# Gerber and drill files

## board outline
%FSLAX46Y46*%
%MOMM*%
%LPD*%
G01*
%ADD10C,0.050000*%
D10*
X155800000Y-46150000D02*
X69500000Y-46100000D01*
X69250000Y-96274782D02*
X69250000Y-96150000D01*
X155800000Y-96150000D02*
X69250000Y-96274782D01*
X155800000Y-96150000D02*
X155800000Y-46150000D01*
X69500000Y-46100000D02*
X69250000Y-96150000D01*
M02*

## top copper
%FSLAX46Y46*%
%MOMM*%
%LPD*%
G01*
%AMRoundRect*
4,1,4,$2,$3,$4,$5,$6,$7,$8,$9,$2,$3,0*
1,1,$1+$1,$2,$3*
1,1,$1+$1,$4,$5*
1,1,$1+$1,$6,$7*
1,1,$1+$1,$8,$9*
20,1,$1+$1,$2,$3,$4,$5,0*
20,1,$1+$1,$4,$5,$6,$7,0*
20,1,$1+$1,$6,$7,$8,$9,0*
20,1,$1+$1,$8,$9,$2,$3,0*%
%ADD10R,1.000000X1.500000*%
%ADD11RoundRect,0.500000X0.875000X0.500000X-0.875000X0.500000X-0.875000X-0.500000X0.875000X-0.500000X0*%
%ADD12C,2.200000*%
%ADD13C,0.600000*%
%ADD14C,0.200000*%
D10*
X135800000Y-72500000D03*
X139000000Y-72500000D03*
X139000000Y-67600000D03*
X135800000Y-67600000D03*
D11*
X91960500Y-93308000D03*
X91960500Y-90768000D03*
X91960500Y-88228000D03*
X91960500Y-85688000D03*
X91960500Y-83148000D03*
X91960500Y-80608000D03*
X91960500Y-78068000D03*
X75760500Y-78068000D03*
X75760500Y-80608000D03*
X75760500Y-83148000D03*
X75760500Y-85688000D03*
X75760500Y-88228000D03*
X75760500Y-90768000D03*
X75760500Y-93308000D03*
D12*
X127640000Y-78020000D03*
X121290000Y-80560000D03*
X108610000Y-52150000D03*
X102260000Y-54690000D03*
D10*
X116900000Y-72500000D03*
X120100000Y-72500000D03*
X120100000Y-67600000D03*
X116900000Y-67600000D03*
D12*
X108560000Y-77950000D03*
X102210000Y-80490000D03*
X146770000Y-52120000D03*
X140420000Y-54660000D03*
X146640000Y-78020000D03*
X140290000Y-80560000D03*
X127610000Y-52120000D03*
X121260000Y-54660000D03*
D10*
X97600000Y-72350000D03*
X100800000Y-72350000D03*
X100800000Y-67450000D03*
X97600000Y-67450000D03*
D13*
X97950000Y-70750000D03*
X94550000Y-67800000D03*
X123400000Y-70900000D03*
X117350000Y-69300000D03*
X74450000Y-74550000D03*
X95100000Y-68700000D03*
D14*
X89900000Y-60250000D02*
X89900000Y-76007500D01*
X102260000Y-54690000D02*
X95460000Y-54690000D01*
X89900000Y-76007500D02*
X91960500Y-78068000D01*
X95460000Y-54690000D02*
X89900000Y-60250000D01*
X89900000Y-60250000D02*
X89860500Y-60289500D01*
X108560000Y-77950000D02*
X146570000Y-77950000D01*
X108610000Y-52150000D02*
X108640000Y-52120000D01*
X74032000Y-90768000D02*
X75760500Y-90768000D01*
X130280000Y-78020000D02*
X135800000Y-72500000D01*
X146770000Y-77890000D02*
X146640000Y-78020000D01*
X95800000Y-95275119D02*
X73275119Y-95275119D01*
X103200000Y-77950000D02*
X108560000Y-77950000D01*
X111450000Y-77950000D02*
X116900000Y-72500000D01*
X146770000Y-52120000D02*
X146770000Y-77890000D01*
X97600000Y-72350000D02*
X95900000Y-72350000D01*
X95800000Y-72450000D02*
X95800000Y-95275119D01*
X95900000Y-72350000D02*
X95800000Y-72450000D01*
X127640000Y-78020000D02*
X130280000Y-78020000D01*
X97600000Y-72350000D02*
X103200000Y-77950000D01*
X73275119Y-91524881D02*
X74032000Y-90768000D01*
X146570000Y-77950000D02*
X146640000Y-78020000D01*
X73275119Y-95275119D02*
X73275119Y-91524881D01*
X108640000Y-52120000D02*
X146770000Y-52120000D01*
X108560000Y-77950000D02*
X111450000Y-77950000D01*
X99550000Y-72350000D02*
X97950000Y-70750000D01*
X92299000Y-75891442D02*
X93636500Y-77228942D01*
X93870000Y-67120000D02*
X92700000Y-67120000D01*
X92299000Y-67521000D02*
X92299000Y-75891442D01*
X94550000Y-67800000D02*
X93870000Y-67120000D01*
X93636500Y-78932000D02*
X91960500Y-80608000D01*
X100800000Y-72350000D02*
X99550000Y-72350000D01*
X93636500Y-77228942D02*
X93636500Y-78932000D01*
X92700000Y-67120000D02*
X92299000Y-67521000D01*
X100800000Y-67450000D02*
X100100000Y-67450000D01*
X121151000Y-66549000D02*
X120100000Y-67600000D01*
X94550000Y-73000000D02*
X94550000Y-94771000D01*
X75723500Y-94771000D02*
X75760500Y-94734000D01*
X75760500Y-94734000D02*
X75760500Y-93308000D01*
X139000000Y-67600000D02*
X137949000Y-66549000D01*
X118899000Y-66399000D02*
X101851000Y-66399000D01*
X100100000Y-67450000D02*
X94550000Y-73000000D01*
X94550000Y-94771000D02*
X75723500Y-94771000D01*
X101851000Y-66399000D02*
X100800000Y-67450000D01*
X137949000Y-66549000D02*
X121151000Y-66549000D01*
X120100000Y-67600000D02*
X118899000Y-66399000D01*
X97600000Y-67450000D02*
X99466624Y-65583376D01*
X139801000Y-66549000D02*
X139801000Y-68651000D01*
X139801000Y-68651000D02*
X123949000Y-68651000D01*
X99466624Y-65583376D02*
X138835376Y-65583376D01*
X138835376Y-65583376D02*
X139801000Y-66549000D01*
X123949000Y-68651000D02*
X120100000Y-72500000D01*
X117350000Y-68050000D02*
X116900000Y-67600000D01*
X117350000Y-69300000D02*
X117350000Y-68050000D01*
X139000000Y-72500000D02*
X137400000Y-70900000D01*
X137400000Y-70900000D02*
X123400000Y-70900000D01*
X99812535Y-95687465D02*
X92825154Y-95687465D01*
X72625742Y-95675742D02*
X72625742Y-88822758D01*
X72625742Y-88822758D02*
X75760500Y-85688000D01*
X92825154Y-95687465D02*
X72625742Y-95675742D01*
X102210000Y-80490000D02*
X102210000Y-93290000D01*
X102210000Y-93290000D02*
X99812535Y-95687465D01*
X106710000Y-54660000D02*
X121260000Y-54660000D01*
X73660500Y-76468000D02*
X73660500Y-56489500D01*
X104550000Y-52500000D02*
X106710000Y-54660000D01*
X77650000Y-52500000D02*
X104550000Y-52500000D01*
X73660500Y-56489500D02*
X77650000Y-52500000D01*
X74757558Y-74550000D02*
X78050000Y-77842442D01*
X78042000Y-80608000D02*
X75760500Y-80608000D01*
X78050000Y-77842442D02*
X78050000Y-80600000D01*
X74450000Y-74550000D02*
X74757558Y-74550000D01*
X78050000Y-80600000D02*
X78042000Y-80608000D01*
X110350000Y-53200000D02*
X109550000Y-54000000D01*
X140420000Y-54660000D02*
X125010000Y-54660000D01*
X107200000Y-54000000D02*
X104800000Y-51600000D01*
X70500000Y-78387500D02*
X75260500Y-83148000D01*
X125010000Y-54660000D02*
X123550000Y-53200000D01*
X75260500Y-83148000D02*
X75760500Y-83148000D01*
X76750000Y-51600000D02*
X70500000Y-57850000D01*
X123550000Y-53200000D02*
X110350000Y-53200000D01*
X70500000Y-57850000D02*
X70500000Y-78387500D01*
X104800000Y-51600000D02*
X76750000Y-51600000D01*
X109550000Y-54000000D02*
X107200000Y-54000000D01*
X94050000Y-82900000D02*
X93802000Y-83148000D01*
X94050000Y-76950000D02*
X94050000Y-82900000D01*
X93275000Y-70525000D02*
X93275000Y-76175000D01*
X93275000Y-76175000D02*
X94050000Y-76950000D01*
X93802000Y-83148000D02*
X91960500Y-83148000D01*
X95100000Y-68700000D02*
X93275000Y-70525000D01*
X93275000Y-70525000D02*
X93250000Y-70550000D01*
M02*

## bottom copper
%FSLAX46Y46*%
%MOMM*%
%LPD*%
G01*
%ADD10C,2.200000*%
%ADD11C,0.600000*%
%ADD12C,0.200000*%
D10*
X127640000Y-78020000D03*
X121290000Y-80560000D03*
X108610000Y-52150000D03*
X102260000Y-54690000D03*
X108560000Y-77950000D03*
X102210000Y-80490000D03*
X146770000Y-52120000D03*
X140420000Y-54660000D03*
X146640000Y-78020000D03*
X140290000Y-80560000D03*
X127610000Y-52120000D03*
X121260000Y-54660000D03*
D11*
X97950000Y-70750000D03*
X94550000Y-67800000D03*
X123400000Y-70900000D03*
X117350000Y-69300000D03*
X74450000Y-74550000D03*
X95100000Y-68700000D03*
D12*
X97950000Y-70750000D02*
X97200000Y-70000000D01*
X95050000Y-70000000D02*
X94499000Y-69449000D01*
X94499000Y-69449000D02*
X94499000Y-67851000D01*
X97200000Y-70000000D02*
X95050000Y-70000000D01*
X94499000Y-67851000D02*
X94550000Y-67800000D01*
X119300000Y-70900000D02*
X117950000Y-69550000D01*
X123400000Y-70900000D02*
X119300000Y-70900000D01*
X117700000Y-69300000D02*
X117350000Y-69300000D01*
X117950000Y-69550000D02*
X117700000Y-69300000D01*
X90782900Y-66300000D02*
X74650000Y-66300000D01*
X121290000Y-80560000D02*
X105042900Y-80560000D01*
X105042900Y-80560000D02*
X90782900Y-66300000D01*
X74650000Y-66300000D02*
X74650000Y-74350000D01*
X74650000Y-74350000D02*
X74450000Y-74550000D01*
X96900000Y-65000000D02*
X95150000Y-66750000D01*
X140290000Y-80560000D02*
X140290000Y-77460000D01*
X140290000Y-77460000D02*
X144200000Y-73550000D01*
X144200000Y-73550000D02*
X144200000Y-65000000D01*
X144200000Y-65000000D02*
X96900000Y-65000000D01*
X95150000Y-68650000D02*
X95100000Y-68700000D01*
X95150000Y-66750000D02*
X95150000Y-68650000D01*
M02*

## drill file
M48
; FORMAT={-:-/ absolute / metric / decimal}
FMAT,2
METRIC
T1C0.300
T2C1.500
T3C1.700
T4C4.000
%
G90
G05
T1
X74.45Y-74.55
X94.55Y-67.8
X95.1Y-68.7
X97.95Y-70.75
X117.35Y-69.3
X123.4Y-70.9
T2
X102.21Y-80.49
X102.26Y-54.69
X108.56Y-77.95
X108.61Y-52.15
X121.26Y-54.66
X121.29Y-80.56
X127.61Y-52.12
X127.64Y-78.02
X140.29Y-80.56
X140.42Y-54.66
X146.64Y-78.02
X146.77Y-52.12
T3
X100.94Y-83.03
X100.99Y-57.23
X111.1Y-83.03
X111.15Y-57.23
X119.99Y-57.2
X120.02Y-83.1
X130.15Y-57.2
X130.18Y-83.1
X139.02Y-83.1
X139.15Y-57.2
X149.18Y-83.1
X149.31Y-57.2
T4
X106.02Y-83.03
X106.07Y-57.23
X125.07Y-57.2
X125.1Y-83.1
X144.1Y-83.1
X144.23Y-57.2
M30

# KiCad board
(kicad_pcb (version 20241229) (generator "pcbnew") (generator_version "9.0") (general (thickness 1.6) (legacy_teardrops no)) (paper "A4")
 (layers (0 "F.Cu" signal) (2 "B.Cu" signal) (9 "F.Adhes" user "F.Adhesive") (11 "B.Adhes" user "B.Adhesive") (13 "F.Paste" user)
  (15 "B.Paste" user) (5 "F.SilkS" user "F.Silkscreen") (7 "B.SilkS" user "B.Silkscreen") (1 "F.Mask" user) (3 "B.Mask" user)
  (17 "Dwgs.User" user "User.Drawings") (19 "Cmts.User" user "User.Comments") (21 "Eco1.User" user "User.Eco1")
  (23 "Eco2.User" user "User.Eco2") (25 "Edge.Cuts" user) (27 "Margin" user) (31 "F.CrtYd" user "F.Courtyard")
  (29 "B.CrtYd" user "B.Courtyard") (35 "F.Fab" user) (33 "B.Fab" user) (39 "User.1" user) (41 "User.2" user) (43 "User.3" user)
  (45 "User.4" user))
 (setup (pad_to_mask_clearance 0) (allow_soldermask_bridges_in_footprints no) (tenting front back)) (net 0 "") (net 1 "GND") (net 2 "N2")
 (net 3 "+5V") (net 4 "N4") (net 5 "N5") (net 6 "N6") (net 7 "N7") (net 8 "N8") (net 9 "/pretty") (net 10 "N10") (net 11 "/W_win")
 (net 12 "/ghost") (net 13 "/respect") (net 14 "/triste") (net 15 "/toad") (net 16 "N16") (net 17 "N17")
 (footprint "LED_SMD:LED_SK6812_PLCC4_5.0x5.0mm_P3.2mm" (layer "F.Cu") (at 137.4 70.05 90)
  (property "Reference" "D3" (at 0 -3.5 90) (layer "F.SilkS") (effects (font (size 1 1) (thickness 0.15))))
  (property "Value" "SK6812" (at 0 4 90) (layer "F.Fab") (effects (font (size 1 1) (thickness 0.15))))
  (pad "1" smd rect (at -2.45 -1.6 270) (size 1.5 1) (layers "F.Cu" "F.Mask" "F.Paste") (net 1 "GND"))
  (pad "2" smd rect (at -2.45 1.6 270) (size 1.5 1) (layers "F.Cu" "F.Mask" "F.Paste") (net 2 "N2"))
  (pad "3" smd rect (at 2.45 1.6 270) (size 1.5 1) (layers "F.Cu" "F.Mask" "F.Paste") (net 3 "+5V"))
  (pad "4" smd rect (at 2.45 -1.6 270) (size 1.5 1) (layers "F.Cu" "F.Mask" "F.Paste") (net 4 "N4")))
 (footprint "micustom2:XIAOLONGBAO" (layer "F.Cu") (at 83.8605 85.688 180)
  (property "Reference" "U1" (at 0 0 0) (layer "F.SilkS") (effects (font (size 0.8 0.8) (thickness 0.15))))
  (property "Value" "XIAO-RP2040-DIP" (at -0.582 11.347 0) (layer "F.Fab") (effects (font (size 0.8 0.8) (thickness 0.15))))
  (pad "1" smd roundrect (at -8.1 -7.62 180) (size 2.75 2) (layers "F.Cu" "F.Mask" "F.Paste") (roundrect_rratio 0.25) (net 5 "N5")
   (solder_mask_margin 0.102))
  (pad "2" smd roundrect (at -8.1 -5.08 180) (size 2.75 2) (layers "F.Cu" "F.Mask" "F.Paste") (roundrect_rratio 0.25) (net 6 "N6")
   (solder_mask_margin 0.102))
  (pad "3" smd roundrect (at -8.1 -2.54 180) (size 2.75 2) (layers "F.Cu" "F.Mask" "F.Paste") (roundrect_rratio 0.25) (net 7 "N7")
   (solder_mask_margin 0.102))
  (pad "4" smd roundrect (at -8.1 0 180) (size 2.75 2) (layers "F.Cu" "F.Mask" "F.Paste") (roundrect_rratio 0.25) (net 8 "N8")
   (solder_mask_margin 0.102))
  (pad "5" smd roundrect (at -8.1 2.54 180) (size 2.75 2) (layers "F.Cu" "F.Mask" "F.Paste") (roundrect_rratio 0.25) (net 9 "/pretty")
   (solder_mask_margin 0.102))
  (pad "6" smd roundrect (at -8.1 5.08 180) (size 2.75 2) (layers "F.Cu" "F.Mask" "F.Paste") (roundrect_rratio 0.25) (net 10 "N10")
   (solder_mask_margin 0.102))
  (pad "7" smd roundrect (at -8.1 7.62 180) (size 2.75 2) (layers "F.Cu" "F.Mask" "F.Paste") (roundrect_rratio 0.25) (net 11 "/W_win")
   (solder_mask_margin 0.102))
  (pad "8" smd roundrect (at 8.1 7.62 180) (size 2.75 2) (layers "F.Cu" "F.Mask" "F.Paste") (roundrect_rratio 0.25) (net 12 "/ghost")
   (solder_mask_margin 0.102))
  (pad "9" smd roundrect (at 8.1 5.08 180) (size 2.75 2) (layers "F.Cu" "F.Mask" "F.Paste") (roundrect_rratio 0.25) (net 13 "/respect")
   (solder_mask_margin 0.102))
  (pad "10" smd roundrect (at 8.1 2.54 180) (size 2.75 2) (layers "F.Cu" "F.Mask" "F.Paste") (roundrect_rratio 0.25) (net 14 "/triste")
   (solder_mask_margin 0.102))
  (pad "11" smd roundrect (at 8.1 0 180) (size 2.75 2) (layers "F.Cu" "F.Mask" "F.Paste") (roundrect_rratio 0.25) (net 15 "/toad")
   (solder_mask_margin 0.102))
  (pad "12" smd roundrect (at 8.1 -2.54 180) (size 2.75 2) (layers "F.Cu" "F.Mask" "F.Paste") (roundrect_rratio 0.25) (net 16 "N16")
   (solder_mask_margin 0.102))
  (pad "13" smd roundrect (at 8.1 -5.08 180) (size 2.75 2) (layers "F.Cu" "F.Mask" "F.Paste") (roundrect_rratio 0.25) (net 1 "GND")
   (solder_mask_margin 0.102))
  (pad "14" smd roundrect (at 8.1 -7.62 180) (size 2.75 2) (layers "F.Cu" "F.Mask" "F.Paste") (roundrect_rratio 0.25) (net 3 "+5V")
   (solder_mask_margin 0.102))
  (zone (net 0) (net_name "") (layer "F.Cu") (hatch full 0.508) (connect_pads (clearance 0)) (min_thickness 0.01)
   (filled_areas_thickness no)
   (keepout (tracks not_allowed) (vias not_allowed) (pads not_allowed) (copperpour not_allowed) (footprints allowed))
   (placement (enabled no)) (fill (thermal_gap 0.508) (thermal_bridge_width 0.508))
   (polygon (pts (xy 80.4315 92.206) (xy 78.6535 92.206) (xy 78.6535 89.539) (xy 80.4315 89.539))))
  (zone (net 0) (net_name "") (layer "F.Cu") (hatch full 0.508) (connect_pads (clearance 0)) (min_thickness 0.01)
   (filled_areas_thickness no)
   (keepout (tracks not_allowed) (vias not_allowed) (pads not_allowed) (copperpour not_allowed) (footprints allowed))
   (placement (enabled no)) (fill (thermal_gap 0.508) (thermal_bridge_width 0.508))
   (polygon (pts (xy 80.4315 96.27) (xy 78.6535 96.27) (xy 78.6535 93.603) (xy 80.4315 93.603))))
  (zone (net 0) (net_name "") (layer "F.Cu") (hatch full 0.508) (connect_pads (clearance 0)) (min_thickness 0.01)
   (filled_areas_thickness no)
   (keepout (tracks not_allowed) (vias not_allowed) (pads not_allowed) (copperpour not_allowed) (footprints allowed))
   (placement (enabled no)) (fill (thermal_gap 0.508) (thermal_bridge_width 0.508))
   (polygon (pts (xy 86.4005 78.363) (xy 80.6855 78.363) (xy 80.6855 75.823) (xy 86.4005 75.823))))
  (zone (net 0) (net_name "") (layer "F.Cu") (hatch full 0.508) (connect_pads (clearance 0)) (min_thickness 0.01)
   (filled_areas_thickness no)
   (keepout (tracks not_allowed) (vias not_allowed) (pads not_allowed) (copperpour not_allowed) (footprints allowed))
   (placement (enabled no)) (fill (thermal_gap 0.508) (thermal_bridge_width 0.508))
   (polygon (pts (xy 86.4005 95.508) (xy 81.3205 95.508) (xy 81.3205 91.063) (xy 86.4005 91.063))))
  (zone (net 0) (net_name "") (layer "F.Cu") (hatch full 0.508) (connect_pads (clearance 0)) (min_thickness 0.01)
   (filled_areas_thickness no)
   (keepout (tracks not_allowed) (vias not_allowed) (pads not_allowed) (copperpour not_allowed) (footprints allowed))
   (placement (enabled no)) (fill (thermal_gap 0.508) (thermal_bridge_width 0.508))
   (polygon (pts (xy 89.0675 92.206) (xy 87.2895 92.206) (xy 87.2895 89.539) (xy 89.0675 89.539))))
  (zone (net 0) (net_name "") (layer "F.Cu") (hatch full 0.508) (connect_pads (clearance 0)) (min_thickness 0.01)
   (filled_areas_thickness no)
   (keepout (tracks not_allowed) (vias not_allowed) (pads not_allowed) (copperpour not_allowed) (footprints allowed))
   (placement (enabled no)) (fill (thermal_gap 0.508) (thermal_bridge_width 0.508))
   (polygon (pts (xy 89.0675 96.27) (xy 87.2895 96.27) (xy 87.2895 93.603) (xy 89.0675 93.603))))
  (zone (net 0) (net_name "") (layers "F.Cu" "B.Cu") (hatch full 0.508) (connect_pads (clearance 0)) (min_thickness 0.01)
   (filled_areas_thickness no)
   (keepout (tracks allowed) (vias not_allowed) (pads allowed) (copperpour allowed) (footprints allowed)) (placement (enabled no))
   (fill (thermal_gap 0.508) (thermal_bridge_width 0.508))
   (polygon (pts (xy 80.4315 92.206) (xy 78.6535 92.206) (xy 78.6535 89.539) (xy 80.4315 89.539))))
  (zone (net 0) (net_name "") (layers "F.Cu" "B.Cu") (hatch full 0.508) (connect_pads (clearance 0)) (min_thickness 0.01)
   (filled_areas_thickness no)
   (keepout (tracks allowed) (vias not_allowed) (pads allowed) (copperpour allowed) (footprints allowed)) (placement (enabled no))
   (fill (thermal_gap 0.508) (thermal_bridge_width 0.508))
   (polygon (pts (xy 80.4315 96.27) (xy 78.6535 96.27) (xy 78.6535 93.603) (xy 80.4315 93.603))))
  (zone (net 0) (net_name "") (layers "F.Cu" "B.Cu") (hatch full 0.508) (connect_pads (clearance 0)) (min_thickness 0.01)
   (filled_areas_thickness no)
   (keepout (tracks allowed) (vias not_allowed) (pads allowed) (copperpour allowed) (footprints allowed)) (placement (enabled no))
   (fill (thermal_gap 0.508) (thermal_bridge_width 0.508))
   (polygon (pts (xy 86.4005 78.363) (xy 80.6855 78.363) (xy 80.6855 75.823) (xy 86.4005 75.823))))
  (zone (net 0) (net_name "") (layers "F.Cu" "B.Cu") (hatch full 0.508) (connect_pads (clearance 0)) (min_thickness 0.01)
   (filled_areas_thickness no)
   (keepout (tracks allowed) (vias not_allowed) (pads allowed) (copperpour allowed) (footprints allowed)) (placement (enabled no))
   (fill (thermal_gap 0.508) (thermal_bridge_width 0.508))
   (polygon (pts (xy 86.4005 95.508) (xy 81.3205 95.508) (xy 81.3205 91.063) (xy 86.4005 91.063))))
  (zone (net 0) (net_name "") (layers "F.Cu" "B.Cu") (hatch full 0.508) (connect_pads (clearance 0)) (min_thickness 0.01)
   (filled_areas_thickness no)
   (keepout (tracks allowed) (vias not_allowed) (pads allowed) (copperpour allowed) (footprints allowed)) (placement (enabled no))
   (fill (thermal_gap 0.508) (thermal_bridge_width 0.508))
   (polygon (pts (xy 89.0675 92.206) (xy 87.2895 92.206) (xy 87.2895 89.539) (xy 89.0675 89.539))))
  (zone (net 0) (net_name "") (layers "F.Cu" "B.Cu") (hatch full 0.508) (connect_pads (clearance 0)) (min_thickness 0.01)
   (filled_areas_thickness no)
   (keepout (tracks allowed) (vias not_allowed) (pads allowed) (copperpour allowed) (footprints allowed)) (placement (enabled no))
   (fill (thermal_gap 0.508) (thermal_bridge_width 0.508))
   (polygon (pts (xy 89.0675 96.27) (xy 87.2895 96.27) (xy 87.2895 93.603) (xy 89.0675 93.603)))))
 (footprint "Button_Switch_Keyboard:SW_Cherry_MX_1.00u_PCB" (layer "F.Cu") (at 127.64 78.02)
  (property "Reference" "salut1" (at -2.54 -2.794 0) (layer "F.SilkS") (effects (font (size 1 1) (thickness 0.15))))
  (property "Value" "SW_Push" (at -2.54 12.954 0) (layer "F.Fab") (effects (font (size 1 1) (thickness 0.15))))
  (pad "" np_thru_hole circle (at -7.62 5.08) (size 1.7 1.7) (drill 1.7) (layers "*.Cu" "*.Mask"))
  (pad "" np_thru_hole circle (at -2.54 5.08) (size 4 4) (drill 4) (layers "*.Cu" "*.Mask"))
  (pad "" np_thru_hole circle (at 2.54 5.08) (size 1.7 1.7) (drill 1.7) (layers "*.Cu" "*.Mask"))
  (pad "1" thru_hole circle (at 0 0) (size 2.2 2.2) (drill 1.5) (layers "*.Cu" "*.Mask") (remove_unused_layers no) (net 1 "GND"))
  (pad "2" thru_hole circle (at -6.35 2.54) (size 2.2 2.2) (drill 1.5) (layers "*.Cu" "*.Mask") (remove_unused_layers no)
   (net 13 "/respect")))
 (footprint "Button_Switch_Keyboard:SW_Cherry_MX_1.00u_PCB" (layer "F.Cu") (at 108.61 52.15)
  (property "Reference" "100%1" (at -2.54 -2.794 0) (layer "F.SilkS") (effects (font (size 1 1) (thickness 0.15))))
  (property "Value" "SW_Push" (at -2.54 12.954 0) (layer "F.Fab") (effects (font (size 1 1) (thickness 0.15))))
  (pad "" np_thru_hole circle (at -7.62 5.08) (size 1.7 1.7) (drill 1.7) (layers "*.Cu" "*.Mask"))
  (pad "" np_thru_hole circle (at -2.54 5.08) (size 4 4) (drill 4) (layers "*.Cu" "*.Mask"))
  (pad "" np_thru_hole circle (at 2.54 5.08) (size 1.7 1.7) (drill 1.7) (layers "*.Cu" "*.Mask"))
  (pad "1" thru_hole circle (at 0 0) (size 2.2 2.2) (drill 1.5) (layers "*.Cu" "*.Mask") (remove_unused_layers no) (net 1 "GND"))
  (pad "2" thru_hole circle (at -6.35 2.54) (size 2.2 2.2) (drill 1.5) (layers "*.Cu" "*.Mask") (remove_unused_layers no) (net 11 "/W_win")))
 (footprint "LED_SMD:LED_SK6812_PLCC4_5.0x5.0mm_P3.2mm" (layer "F.Cu") (at 118.5 70.05 90)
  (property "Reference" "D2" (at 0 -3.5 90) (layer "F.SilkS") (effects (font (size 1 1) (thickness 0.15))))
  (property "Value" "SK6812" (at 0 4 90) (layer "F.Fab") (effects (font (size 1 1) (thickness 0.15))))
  (pad "1" smd rect (at -2.45 -1.6 270) (size 1.5 1) (layers "F.Cu" "F.Mask" "F.Paste") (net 1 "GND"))
  (pad "2" smd rect (at -2.45 1.6 270) (size 1.5 1) (layers "F.Cu" "F.Mask" "F.Paste") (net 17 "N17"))
  (pad "3" smd rect (at 2.45 1.6 270) (size 1.5 1) (layers "F.Cu" "F.Mask" "F.Paste") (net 3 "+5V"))
  (pad "4" smd rect (at 2.45 -1.6 270) (size 1.5 1) (layers "F.Cu" "F.Mask" "F.Paste") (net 2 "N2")))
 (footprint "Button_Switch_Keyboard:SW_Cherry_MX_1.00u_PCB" (layer "F.Cu") (at 108.56 77.95)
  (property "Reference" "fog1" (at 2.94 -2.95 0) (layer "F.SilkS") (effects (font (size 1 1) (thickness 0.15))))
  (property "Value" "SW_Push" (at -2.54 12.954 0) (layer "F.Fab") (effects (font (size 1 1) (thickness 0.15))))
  (pad "" np_thru_hole circle (at -7.62 5.08) (size 1.7 1.7) (drill 1.7) (layers "*.Cu" "*.Mask"))
  (pad "" np_thru_hole circle (at -2.54 5.08) (size 4 4) (drill 4) (layers "*.Cu" "*.Mask"))
  (pad "" np_thru_hole circle (at 2.54 5.08) (size 1.7 1.7) (drill 1.7) (layers "*.Cu" "*.Mask"))
  (pad "1" thru_hole circle (at 0 0) (size 2.2 2.2) (drill 1.5) (layers "*.Cu" "*.Mask") (remove_unused_layers no) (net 1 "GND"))
  (pad "2" thru_hole circle (at -6.35 2.54) (size 2.2 2.2) (drill 1.5) (layers "*.Cu" "*.Mask") (remove_unused_layers no) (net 15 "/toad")))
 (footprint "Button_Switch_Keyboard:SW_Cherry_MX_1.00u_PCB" (layer "F.Cu") (at 146.77 52.12)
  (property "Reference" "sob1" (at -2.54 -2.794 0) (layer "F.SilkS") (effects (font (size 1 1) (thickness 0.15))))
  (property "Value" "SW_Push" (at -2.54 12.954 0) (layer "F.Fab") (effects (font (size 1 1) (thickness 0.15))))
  (pad "" np_thru_hole circle (at -7.62 5.08) (size 1.7 1.7) (drill 1.7) (layers "*.Cu" "*.Mask"))
  (pad "" np_thru_hole circle (at -2.54 5.08) (size 4 4) (drill 4) (layers "*.Cu" "*.Mask"))
  (pad "" np_thru_hole circle (at 2.54 5.08) (size 1.7 1.7) (drill 1.7) (layers "*.Cu" "*.Mask"))
  (pad "1" thru_hole circle (at 0 0) (size 2.2 2.2) (drill 1.5) (layers "*.Cu" "*.Mask") (remove_unused_layers no) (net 1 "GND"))
  (pad "2" thru_hole circle (at -6.35 2.54) (size 2.2 2.2) (drill 1.5) (layers "*.Cu" "*.Mask") (remove_unused_layers no) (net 14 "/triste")))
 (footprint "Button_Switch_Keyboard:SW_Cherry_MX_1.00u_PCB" (layer "F.Cu") (at 146.64 78.02)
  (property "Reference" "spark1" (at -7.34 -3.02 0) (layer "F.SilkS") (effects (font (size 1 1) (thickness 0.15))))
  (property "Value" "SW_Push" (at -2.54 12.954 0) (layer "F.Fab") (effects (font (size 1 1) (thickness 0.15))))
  (pad "" np_thru_hole circle (at -7.62 5.08) (size 1.7 1.7) (drill 1.7) (layers "*.Cu" "*.Mask"))
  (pad "" np_thru_hole circle (at -2.54 5.08) (size 4 4) (drill 4) (layers "*.Cu" "*.Mask"))
  (pad "" np_thru_hole circle (at 2.54 5.08) (size 1.7 1.7) (drill 1.7) (layers "*.Cu" "*.Mask"))
  (pad "1" thru_hole circle (at 0 0) (size 2.2 2.2) (drill 1.5) (layers "*.Cu" "*.Mask") (remove_unused_layers no) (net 1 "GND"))
  (pad "2" thru_hole circle (at -6.35 2.54) (size 2.2 2.2) (drill 1.5) (layers "*.Cu" "*.Mask") (remove_unused_layers no) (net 9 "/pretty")))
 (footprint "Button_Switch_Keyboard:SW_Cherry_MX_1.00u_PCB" (layer "F.Cu") (at 127.61 52.12)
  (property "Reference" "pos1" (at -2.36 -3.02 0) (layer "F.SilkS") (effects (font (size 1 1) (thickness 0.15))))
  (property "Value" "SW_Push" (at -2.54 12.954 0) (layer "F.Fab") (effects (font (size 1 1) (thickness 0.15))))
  (pad "" np_thru_hole circle (at -7.62 5.08) (size 1.7 1.7) (drill 1.7) (layers "*.Cu" "*.Mask"))
  (pad "" np_thru_hole circle (at -2.54 5.08) (size 4 4) (drill 4) (layers "*.Cu" "*.Mask"))
  (pad "" np_thru_hole circle (at 2.54 5.08) (size 1.7 1.7) (drill 1.7) (layers "*.Cu" "*.Mask"))
  (pad "1" thru_hole circle (at 0 0) (size 2.2 2.2) (drill 1.5) (layers "*.Cu" "*.Mask") (remove_unused_layers no) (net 1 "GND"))
  (pad "2" thru_hole circle (at -6.35 2.54) (size 2.2 2.2) (drill 1.5) (layers "*.Cu" "*.Mask") (remove_unused_layers no) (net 12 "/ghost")))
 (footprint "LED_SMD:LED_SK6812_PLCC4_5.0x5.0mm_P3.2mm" (layer "F.Cu") (at 99.2 69.9 90)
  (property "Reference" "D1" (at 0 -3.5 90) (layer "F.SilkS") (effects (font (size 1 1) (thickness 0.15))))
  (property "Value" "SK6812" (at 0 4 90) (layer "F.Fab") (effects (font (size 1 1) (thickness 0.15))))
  (pad "1" smd rect (at -2.45 -1.6 270) (size 1.5 1) (layers "F.Cu" "F.Mask" "F.Paste") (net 1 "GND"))
  (pad "2" smd rect (at -2.45 1.6 270) (size 1.5 1) (layers "F.Cu" "F.Mask" "F.Paste") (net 10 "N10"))
  (pad "3" smd rect (at 2.45 1.6 270) (size 1.5 1) (layers "F.Cu" "F.Mask" "F.Paste") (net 3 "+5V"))
  (pad "4" smd rect (at 2.45 -1.6 270) (size 1.5 1) (layers "F.Cu" "F.Mask" "F.Paste") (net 17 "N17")))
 (gr_line (start 155.8 46.15) (end 69.5 46.1) (stroke (width 0.05) (type default)) (layer "Edge.Cuts"))
 (gr_line (start 69.25 96.274782) (end 69.25 96.15) (stroke (width 0.05) (type default)) (layer "Edge.Cuts"))
 (gr_line (start 155.8 96.15) (end 69.25 96.274782) (stroke (width 0.05) (type default)) (layer "Edge.Cuts"))
 (gr_line (start 155.8 96.15) (end 155.8 46.15) (stroke (width 0.05) (type default)) (layer "Edge.Cuts"))
 (gr_line (start 69.5 46.1) (end 69.25 96.15) (stroke (width 0.05) (type default)) (layer "Edge.Cuts"))
 (segment (start 89.9 60.25) (end 89.9 76.0075) (width 0.2) (layer "F.Cu") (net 11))
 (segment (start 102.26 54.69) (end 95.46 54.69) (width 0.2) (layer "F.Cu") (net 11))
 (segment (start 89.9 76.0075) (end 91.9605 78.068) (width 0.2) (layer "F.Cu") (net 11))
 (segment (start 95.46 54.69) (end 89.9 60.25) (width 0.2) (layer "F.Cu") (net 11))
 (segment (start 89.9 60.25) (end 89.8605 60.2895) (width 0.2) (layer "F.Cu") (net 11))
 (segment (start 108.56 77.95) (end 146.57 77.95) (width 0.2) (layer "F.Cu") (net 1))
 (segment (start 108.61 52.15) (end 108.64 52.12) (width 0.2) (layer "F.Cu") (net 1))
 (segment (start 74.032 90.768) (end 75.7605 90.768) (width 0.2) (layer "F.Cu") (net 1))
 (segment (start 130.28 78.02) (end 135.8 72.5) (width 0.2) (layer "F.Cu") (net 1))
 (segment (start 146.77 77.89) (end 146.64 78.02) (width 0.2) (layer "F.Cu") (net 1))
 (segment (start 95.8 95.275119) (end 73.275119 95.275119) (width 0.2) (layer "F.Cu") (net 1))
 (segment (start 103.2 77.95) (end 108.56 77.95) (width 0.2) (layer "F.Cu") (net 1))
 (segment (start 111.45 77.95) (end 116.9 72.5) (width 0.2) (layer "F.Cu") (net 1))
 (segment (start 146.77 52.12) (end 146.77 77.89) (width 0.2) (layer "F.Cu") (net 1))
 (segment (start 97.6 72.35) (end 95.9 72.35) (width 0.2) (layer "F.Cu") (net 1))
 (segment (start 95.8 72.45) (end 95.8 95.275119) (width 0.2) (layer "F.Cu") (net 1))
 (segment (start 95.9 72.35) (end 95.8 72.45) (width 0.2) (layer "F.Cu") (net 1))
 (segment (start 127.64 78.02) (end 130.28 78.02) (width 0.2) (layer "F.Cu") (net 1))
 (segment (start 97.6 72.35) (end 103.2 77.95) (width 0.2) (layer "F.Cu") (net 1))
 (segment (start 73.275119 91.524881) (end 74.032 90.768) (width 0.2) (layer "F.Cu") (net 1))
 (segment (start 146.57 77.95) (end 146.64 78.02) (width 0.2) (layer "F.Cu") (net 1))
 (segment (start 73.275119 95.275119) (end 73.275119 91.524881) (width 0.2) (layer "F.Cu") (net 1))
 (segment (start 108.64 52.12) (end 146.77 52.12) (width 0.2) (layer "F.Cu") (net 1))
 (segment (start 108.56 77.95) (end 111.45 77.95) (width 0.2) (layer "F.Cu") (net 1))
 (segment (start 99.55 72.35) (end 97.95 70.75) (width 0.2) (layer "F.Cu") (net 10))
 (segment (start 92.299 75.891442) (end 93.6365 77.228942) (width 0.2) (layer "F.Cu") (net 10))
 (segment (start 93.87 67.12) (end 92.7 67.12) (width 0.2) (layer "F.Cu") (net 10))
 (segment (start 92.299 67.521) (end 92.299 75.891442) (width 0.2) (layer "F.Cu") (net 10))
 (segment (start 94.55 67.8) (end 93.87 67.12) (width 0.2) (layer "F.Cu") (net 10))
 (segment (start 93.6365 78.932) (end 91.9605 80.608) (width 0.2) (layer "F.Cu") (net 10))
 (segment (start 100.8 72.35) (end 99.55 72.35) (width 0.2) (layer "F.Cu") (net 10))
 (segment (start 93.6365 77.228942) (end 93.6365 78.932) (width 0.2) (layer "F.Cu") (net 10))
 (segment (start 92.7 67.12) (end 92.299 67.521) (width 0.2) (layer "F.Cu") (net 10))
 (via (at 97.95 70.75) (size 0.6) (drill 0.3) (layers "F.Cu" "B.Cu") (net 10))
 (via (at 94.55 67.8) (size 0.6) (drill 0.3) (layers "F.Cu" "B.Cu") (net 10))
 (segment (start 97.95 70.75) (end 97.2 70) (width 0.2) (layer "B.Cu") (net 10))
 (segment (start 95.05 70) (end 94.499 69.449) (width 0.2) (layer "B.Cu") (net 10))
 (segment (start 94.499 69.449) (end 94.499 67.851) (width 0.2) (layer "B.Cu") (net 10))
 (segment (start 97.2 70) (end 95.05 70) (width 0.2) (layer "B.Cu") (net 10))
 (segment (start 94.499 67.851) (end 94.55 67.8) (width 0.2) (layer "B.Cu") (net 10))
 (segment (start 100.8 67.45) (end 100.1 67.45) (width 0.2) (layer "F.Cu") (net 3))
 (segment (start 121.151 66.549) (end 120.1 67.6) (width 0.2) (layer "F.Cu") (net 3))
 (segment (start 94.55 73) (end 94.55 94.771) (width 0.2) (layer "F.Cu") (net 3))
 (segment (start 75.7235 94.771) (end 75.7605 94.734) (width 0.2) (layer "F.Cu") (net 3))
 (segment (start 75.7605 94.734) (end 75.7605 93.308) (width 0.2) (layer "F.Cu") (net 3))
 (segment (start 139 67.6) (end 137.949 66.549) (width 0.2) (layer "F.Cu") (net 3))
 (segment (start 118.899 66.399) (end 101.851 66.399) (width 0.2) (layer "F.Cu") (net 3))
 (segment (start 100.1 67.45) (end 94.55 73) (width 0.2) (layer "F.Cu") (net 3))
 (segment (start 94.55 94.771) (end 75.7235 94.771) (width 0.2) (layer "F.Cu") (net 3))
 (segment (start 101.851 66.399) (end 100.8 67.45) (width 0.2) (layer "F.Cu") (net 3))
 (segment (start 137.949 66.549) (end 121.151 66.549) (width 0.2) (layer "F.Cu") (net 3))
 (segment (start 120.1 67.6) (end 118.899 66.399) (width 0.2) (layer "F.Cu") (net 3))
 (segment (start 97.6 67.45) (end 99.466624 65.583376) (width 0.2) (layer "F.Cu") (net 17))
 (segment (start 139.801 66.549) (end 139.801 68.651) (width 0.2) (layer "F.Cu") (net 17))
 (segment (start 139.801 68.651) (end 123.949 68.651) (width 0.2) (layer "F.Cu") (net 17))
 (segment (start 99.466624 65.583376) (end 138.835376 65.583376) (width 0.2) (layer "F.Cu") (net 17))
 (segment (start 138.835376 65.583376) (end 139.801 66.549) (width 0.2) (layer "F.Cu") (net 17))
 (segment (start 123.949 68.651) (end 120.1 72.5) (width 0.2) (layer "F.Cu") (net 17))
 (segment (start 117.35 68.05) (end 116.9 67.6) (width 0.2) (layer "F.Cu") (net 2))
 (segment (start 117.35 69.3) (end 117.35 68.05) (width 0.2) (layer "F.Cu") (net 2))
 (segment (start 139 72.5) (end 137.4 70.9) (width 0.2) (layer "F.Cu") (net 2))
 (segment (start 137.4 70.9) (end 123.4 70.9) (width 0.2) (layer "F.Cu") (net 2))
 (via (at 123.4 70.9) (size 0.6) (drill 0.3) (layers "F.Cu" "B.Cu") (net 2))
 (via (at 117.35 69.3) (size 0.6) (drill 0.3) (layers "F.Cu" "B.Cu") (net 2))
 (segment (start 119.3 70.9) (end 117.95 69.55) (width 0.2) (layer "B.Cu") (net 2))
 (segment (start 123.4 70.9) (end 119.3 70.9) (width 0.2) (layer "B.Cu") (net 2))
 (segment (start 117.7 69.3) (end 117.35 69.3) (width 0.2) (layer "B.Cu") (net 2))
 (segment (start 117.95 69.55) (end 117.7 69.3) (width 0.2) (layer "B.Cu") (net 2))
 (segment (start 99.812535 95.687465) (end 92.825154 95.687465) (width 0.2) (layer "F.Cu") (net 15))
 (segment (start 72.625742 95.675742) (end 72.625742 88.822758) (width 0.2) (layer "F.Cu") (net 15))
 (segment (start 72.625742 88.822758) (end 75.7605 85.688) (width 0.2) (layer "F.Cu") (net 15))
 (segment (start 92.825154 95.687465) (end 72.625742 95.675742) (width 0.2) (layer "F.Cu") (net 15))
 (segment (start 102.21 80.49) (end 102.21 93.29) (width 0.2) (layer "F.Cu") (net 15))
 (segment (start 102.21 93.29) (end 99.812535 95.687465) (width 0.2) (layer "F.Cu") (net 15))
 (segment (start 106.71 54.66) (end 121.26 54.66) (width 0.2) (layer "F.Cu") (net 12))
 (segment (start 73.6605 76.468) (end 73.6605 56.4895) (width 0.2) (layer "F.Cu") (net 12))
 (segment (start 104.55 52.5) (end 106.71 54.66) (width 0.2) (layer "F.Cu") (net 12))
 (segment (start 77.65 52.5) (end 104.55 52.5) (width 0.2) (layer "F.Cu") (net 12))
 (segment (start 73.6605 56.4895) (end 77.65 52.5) (width 0.2) (layer "F.Cu") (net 12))
 (segment (start 74.757558 74.55) (end 78.05 77.842442) (width 0.2) (layer "F.Cu") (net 13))
 (segment (start 78.042 80.608) (end 75.7605 80.608) (width 0.2) (layer "F.Cu") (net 13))
 (segment (start 78.05 77.842442) (end 78.05 80.6) (width 0.2) (layer "F.Cu") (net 13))
 (segment (start 74.45 74.55) (end 74.757558 74.55) (width 0.2) (layer "F.Cu") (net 13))
 (segment (start 78.05 80.6) (end 78.042 80.608) (width 0.2) (layer "F.Cu") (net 13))
 (via (at 74.45 74.55) (size 0.6) (drill 0.3) (layers "F.Cu" "B.Cu") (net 13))
 (segment (start 90.7829 66.3) (end 74.65 66.3) (width 0.2) (layer "B.Cu") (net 13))
 (segment (start 121.29 80.56) (end 105.0429 80.56) (width 0.2) (layer "B.Cu") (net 13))
 (segment (start 105.0429 80.56) (end 90.7829 66.3) (width 0.2) (layer "B.Cu") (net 13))
 (segment (start 74.65 66.3) (end 74.65 74.35) (width 0.2) (layer "B.Cu") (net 13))
 (segment (start 74.65 74.35) (end 74.45 74.55) (width 0.2) (layer "B.Cu") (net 13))
 (segment (start 110.35 53.2) (end 109.55 54) (width 0.2) (layer "F.Cu") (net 14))
 (segment (start 140.42 54.66) (end 125.01 54.66) (width 0.2) (layer "F.Cu") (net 14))
 (segment (start 107.2 54) (end 104.8 51.6) (width 0.2) (layer "F.Cu") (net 14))
 (segment (start 70.5 78.3875) (end 75.2605 83.148) (width 0.2) (layer "F.Cu") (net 14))
 (segment (start 125.01 54.66) (end 123.55 53.2) (width 0.2) (layer "F.Cu") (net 14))
 (segment (start 75.2605 83.148) (end 75.7605 83.148) (width 0.2) (layer "F.Cu") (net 14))
 (segment (start 76.75 51.6) (end 70.5 57.85) (width 0.2) (layer "F.Cu") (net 14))
 (segment (start 123.55 53.2) (end 110.35 53.2) (width 0.2) (layer "F.Cu") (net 14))
 (segment (start 70.5 57.85) (end 70.5 78.3875) (width 0.2) (layer "F.Cu") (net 14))
 (segment (start 104.8 51.6) (end 76.75 51.6) (width 0.2) (layer "F.Cu") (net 14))
 (segment (start 109.55 54) (end 107.2 54) (width 0.2) (layer "F.Cu") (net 14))
 (segment (start 94.05 82.9) (end 93.802 83.148) (width 0.2) (layer "F.Cu") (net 9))
 (segment (start 94.05 76.95) (end 94.05 82.9) (width 0.2) (layer "F.Cu") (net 9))
 (segment (start 93.275 70.525) (end 93.275 76.175) (width 0.2) (layer "F.Cu") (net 9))
 (segment (start 93.275 76.175) (end 94.05 76.95) (width 0.2) (layer "F.Cu") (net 9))
 (segment (start 93.802 83.148) (end 91.9605 83.148) (width 0.2) (layer "F.Cu") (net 9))
 (segment (start 95.1 68.7) (end 93.275 70.525) (width 0.2) (layer "F.Cu") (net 9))
 (segment (start 93.275 70.525) (end 93.25 70.55) (width 0.2) (layer "F.Cu") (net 9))
 (via (at 95.1 68.7) (size 0.6) (drill 0.3) (layers "F.Cu" "B.Cu") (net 9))
 (segment (start 96.9 65) (end 95.15 66.75) (width 0.2) (layer "B.Cu") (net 9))
 (segment (start 140.29 80.56) (end 140.29 77.46) (width 0.2) (layer "B.Cu") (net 9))
 (segment (start 140.29 77.46) (end 144.2 73.55) (width 0.2) (layer "B.Cu") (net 9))
 (segment (start 144.2 73.55) (end 144.2 65) (width 0.2) (layer "B.Cu") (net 9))
 (segment (start 144.2 65) (end 96.9 65) (width 0.2) (layer "B.Cu") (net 9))
 (segment (start 95.15 68.65) (end 95.1 68.7) (width 0.2) (layer "B.Cu") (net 9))
 (segment (start 95.15 66.75) (end 95.15 68.65) (width 0.2) (layer "B.Cu") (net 9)))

